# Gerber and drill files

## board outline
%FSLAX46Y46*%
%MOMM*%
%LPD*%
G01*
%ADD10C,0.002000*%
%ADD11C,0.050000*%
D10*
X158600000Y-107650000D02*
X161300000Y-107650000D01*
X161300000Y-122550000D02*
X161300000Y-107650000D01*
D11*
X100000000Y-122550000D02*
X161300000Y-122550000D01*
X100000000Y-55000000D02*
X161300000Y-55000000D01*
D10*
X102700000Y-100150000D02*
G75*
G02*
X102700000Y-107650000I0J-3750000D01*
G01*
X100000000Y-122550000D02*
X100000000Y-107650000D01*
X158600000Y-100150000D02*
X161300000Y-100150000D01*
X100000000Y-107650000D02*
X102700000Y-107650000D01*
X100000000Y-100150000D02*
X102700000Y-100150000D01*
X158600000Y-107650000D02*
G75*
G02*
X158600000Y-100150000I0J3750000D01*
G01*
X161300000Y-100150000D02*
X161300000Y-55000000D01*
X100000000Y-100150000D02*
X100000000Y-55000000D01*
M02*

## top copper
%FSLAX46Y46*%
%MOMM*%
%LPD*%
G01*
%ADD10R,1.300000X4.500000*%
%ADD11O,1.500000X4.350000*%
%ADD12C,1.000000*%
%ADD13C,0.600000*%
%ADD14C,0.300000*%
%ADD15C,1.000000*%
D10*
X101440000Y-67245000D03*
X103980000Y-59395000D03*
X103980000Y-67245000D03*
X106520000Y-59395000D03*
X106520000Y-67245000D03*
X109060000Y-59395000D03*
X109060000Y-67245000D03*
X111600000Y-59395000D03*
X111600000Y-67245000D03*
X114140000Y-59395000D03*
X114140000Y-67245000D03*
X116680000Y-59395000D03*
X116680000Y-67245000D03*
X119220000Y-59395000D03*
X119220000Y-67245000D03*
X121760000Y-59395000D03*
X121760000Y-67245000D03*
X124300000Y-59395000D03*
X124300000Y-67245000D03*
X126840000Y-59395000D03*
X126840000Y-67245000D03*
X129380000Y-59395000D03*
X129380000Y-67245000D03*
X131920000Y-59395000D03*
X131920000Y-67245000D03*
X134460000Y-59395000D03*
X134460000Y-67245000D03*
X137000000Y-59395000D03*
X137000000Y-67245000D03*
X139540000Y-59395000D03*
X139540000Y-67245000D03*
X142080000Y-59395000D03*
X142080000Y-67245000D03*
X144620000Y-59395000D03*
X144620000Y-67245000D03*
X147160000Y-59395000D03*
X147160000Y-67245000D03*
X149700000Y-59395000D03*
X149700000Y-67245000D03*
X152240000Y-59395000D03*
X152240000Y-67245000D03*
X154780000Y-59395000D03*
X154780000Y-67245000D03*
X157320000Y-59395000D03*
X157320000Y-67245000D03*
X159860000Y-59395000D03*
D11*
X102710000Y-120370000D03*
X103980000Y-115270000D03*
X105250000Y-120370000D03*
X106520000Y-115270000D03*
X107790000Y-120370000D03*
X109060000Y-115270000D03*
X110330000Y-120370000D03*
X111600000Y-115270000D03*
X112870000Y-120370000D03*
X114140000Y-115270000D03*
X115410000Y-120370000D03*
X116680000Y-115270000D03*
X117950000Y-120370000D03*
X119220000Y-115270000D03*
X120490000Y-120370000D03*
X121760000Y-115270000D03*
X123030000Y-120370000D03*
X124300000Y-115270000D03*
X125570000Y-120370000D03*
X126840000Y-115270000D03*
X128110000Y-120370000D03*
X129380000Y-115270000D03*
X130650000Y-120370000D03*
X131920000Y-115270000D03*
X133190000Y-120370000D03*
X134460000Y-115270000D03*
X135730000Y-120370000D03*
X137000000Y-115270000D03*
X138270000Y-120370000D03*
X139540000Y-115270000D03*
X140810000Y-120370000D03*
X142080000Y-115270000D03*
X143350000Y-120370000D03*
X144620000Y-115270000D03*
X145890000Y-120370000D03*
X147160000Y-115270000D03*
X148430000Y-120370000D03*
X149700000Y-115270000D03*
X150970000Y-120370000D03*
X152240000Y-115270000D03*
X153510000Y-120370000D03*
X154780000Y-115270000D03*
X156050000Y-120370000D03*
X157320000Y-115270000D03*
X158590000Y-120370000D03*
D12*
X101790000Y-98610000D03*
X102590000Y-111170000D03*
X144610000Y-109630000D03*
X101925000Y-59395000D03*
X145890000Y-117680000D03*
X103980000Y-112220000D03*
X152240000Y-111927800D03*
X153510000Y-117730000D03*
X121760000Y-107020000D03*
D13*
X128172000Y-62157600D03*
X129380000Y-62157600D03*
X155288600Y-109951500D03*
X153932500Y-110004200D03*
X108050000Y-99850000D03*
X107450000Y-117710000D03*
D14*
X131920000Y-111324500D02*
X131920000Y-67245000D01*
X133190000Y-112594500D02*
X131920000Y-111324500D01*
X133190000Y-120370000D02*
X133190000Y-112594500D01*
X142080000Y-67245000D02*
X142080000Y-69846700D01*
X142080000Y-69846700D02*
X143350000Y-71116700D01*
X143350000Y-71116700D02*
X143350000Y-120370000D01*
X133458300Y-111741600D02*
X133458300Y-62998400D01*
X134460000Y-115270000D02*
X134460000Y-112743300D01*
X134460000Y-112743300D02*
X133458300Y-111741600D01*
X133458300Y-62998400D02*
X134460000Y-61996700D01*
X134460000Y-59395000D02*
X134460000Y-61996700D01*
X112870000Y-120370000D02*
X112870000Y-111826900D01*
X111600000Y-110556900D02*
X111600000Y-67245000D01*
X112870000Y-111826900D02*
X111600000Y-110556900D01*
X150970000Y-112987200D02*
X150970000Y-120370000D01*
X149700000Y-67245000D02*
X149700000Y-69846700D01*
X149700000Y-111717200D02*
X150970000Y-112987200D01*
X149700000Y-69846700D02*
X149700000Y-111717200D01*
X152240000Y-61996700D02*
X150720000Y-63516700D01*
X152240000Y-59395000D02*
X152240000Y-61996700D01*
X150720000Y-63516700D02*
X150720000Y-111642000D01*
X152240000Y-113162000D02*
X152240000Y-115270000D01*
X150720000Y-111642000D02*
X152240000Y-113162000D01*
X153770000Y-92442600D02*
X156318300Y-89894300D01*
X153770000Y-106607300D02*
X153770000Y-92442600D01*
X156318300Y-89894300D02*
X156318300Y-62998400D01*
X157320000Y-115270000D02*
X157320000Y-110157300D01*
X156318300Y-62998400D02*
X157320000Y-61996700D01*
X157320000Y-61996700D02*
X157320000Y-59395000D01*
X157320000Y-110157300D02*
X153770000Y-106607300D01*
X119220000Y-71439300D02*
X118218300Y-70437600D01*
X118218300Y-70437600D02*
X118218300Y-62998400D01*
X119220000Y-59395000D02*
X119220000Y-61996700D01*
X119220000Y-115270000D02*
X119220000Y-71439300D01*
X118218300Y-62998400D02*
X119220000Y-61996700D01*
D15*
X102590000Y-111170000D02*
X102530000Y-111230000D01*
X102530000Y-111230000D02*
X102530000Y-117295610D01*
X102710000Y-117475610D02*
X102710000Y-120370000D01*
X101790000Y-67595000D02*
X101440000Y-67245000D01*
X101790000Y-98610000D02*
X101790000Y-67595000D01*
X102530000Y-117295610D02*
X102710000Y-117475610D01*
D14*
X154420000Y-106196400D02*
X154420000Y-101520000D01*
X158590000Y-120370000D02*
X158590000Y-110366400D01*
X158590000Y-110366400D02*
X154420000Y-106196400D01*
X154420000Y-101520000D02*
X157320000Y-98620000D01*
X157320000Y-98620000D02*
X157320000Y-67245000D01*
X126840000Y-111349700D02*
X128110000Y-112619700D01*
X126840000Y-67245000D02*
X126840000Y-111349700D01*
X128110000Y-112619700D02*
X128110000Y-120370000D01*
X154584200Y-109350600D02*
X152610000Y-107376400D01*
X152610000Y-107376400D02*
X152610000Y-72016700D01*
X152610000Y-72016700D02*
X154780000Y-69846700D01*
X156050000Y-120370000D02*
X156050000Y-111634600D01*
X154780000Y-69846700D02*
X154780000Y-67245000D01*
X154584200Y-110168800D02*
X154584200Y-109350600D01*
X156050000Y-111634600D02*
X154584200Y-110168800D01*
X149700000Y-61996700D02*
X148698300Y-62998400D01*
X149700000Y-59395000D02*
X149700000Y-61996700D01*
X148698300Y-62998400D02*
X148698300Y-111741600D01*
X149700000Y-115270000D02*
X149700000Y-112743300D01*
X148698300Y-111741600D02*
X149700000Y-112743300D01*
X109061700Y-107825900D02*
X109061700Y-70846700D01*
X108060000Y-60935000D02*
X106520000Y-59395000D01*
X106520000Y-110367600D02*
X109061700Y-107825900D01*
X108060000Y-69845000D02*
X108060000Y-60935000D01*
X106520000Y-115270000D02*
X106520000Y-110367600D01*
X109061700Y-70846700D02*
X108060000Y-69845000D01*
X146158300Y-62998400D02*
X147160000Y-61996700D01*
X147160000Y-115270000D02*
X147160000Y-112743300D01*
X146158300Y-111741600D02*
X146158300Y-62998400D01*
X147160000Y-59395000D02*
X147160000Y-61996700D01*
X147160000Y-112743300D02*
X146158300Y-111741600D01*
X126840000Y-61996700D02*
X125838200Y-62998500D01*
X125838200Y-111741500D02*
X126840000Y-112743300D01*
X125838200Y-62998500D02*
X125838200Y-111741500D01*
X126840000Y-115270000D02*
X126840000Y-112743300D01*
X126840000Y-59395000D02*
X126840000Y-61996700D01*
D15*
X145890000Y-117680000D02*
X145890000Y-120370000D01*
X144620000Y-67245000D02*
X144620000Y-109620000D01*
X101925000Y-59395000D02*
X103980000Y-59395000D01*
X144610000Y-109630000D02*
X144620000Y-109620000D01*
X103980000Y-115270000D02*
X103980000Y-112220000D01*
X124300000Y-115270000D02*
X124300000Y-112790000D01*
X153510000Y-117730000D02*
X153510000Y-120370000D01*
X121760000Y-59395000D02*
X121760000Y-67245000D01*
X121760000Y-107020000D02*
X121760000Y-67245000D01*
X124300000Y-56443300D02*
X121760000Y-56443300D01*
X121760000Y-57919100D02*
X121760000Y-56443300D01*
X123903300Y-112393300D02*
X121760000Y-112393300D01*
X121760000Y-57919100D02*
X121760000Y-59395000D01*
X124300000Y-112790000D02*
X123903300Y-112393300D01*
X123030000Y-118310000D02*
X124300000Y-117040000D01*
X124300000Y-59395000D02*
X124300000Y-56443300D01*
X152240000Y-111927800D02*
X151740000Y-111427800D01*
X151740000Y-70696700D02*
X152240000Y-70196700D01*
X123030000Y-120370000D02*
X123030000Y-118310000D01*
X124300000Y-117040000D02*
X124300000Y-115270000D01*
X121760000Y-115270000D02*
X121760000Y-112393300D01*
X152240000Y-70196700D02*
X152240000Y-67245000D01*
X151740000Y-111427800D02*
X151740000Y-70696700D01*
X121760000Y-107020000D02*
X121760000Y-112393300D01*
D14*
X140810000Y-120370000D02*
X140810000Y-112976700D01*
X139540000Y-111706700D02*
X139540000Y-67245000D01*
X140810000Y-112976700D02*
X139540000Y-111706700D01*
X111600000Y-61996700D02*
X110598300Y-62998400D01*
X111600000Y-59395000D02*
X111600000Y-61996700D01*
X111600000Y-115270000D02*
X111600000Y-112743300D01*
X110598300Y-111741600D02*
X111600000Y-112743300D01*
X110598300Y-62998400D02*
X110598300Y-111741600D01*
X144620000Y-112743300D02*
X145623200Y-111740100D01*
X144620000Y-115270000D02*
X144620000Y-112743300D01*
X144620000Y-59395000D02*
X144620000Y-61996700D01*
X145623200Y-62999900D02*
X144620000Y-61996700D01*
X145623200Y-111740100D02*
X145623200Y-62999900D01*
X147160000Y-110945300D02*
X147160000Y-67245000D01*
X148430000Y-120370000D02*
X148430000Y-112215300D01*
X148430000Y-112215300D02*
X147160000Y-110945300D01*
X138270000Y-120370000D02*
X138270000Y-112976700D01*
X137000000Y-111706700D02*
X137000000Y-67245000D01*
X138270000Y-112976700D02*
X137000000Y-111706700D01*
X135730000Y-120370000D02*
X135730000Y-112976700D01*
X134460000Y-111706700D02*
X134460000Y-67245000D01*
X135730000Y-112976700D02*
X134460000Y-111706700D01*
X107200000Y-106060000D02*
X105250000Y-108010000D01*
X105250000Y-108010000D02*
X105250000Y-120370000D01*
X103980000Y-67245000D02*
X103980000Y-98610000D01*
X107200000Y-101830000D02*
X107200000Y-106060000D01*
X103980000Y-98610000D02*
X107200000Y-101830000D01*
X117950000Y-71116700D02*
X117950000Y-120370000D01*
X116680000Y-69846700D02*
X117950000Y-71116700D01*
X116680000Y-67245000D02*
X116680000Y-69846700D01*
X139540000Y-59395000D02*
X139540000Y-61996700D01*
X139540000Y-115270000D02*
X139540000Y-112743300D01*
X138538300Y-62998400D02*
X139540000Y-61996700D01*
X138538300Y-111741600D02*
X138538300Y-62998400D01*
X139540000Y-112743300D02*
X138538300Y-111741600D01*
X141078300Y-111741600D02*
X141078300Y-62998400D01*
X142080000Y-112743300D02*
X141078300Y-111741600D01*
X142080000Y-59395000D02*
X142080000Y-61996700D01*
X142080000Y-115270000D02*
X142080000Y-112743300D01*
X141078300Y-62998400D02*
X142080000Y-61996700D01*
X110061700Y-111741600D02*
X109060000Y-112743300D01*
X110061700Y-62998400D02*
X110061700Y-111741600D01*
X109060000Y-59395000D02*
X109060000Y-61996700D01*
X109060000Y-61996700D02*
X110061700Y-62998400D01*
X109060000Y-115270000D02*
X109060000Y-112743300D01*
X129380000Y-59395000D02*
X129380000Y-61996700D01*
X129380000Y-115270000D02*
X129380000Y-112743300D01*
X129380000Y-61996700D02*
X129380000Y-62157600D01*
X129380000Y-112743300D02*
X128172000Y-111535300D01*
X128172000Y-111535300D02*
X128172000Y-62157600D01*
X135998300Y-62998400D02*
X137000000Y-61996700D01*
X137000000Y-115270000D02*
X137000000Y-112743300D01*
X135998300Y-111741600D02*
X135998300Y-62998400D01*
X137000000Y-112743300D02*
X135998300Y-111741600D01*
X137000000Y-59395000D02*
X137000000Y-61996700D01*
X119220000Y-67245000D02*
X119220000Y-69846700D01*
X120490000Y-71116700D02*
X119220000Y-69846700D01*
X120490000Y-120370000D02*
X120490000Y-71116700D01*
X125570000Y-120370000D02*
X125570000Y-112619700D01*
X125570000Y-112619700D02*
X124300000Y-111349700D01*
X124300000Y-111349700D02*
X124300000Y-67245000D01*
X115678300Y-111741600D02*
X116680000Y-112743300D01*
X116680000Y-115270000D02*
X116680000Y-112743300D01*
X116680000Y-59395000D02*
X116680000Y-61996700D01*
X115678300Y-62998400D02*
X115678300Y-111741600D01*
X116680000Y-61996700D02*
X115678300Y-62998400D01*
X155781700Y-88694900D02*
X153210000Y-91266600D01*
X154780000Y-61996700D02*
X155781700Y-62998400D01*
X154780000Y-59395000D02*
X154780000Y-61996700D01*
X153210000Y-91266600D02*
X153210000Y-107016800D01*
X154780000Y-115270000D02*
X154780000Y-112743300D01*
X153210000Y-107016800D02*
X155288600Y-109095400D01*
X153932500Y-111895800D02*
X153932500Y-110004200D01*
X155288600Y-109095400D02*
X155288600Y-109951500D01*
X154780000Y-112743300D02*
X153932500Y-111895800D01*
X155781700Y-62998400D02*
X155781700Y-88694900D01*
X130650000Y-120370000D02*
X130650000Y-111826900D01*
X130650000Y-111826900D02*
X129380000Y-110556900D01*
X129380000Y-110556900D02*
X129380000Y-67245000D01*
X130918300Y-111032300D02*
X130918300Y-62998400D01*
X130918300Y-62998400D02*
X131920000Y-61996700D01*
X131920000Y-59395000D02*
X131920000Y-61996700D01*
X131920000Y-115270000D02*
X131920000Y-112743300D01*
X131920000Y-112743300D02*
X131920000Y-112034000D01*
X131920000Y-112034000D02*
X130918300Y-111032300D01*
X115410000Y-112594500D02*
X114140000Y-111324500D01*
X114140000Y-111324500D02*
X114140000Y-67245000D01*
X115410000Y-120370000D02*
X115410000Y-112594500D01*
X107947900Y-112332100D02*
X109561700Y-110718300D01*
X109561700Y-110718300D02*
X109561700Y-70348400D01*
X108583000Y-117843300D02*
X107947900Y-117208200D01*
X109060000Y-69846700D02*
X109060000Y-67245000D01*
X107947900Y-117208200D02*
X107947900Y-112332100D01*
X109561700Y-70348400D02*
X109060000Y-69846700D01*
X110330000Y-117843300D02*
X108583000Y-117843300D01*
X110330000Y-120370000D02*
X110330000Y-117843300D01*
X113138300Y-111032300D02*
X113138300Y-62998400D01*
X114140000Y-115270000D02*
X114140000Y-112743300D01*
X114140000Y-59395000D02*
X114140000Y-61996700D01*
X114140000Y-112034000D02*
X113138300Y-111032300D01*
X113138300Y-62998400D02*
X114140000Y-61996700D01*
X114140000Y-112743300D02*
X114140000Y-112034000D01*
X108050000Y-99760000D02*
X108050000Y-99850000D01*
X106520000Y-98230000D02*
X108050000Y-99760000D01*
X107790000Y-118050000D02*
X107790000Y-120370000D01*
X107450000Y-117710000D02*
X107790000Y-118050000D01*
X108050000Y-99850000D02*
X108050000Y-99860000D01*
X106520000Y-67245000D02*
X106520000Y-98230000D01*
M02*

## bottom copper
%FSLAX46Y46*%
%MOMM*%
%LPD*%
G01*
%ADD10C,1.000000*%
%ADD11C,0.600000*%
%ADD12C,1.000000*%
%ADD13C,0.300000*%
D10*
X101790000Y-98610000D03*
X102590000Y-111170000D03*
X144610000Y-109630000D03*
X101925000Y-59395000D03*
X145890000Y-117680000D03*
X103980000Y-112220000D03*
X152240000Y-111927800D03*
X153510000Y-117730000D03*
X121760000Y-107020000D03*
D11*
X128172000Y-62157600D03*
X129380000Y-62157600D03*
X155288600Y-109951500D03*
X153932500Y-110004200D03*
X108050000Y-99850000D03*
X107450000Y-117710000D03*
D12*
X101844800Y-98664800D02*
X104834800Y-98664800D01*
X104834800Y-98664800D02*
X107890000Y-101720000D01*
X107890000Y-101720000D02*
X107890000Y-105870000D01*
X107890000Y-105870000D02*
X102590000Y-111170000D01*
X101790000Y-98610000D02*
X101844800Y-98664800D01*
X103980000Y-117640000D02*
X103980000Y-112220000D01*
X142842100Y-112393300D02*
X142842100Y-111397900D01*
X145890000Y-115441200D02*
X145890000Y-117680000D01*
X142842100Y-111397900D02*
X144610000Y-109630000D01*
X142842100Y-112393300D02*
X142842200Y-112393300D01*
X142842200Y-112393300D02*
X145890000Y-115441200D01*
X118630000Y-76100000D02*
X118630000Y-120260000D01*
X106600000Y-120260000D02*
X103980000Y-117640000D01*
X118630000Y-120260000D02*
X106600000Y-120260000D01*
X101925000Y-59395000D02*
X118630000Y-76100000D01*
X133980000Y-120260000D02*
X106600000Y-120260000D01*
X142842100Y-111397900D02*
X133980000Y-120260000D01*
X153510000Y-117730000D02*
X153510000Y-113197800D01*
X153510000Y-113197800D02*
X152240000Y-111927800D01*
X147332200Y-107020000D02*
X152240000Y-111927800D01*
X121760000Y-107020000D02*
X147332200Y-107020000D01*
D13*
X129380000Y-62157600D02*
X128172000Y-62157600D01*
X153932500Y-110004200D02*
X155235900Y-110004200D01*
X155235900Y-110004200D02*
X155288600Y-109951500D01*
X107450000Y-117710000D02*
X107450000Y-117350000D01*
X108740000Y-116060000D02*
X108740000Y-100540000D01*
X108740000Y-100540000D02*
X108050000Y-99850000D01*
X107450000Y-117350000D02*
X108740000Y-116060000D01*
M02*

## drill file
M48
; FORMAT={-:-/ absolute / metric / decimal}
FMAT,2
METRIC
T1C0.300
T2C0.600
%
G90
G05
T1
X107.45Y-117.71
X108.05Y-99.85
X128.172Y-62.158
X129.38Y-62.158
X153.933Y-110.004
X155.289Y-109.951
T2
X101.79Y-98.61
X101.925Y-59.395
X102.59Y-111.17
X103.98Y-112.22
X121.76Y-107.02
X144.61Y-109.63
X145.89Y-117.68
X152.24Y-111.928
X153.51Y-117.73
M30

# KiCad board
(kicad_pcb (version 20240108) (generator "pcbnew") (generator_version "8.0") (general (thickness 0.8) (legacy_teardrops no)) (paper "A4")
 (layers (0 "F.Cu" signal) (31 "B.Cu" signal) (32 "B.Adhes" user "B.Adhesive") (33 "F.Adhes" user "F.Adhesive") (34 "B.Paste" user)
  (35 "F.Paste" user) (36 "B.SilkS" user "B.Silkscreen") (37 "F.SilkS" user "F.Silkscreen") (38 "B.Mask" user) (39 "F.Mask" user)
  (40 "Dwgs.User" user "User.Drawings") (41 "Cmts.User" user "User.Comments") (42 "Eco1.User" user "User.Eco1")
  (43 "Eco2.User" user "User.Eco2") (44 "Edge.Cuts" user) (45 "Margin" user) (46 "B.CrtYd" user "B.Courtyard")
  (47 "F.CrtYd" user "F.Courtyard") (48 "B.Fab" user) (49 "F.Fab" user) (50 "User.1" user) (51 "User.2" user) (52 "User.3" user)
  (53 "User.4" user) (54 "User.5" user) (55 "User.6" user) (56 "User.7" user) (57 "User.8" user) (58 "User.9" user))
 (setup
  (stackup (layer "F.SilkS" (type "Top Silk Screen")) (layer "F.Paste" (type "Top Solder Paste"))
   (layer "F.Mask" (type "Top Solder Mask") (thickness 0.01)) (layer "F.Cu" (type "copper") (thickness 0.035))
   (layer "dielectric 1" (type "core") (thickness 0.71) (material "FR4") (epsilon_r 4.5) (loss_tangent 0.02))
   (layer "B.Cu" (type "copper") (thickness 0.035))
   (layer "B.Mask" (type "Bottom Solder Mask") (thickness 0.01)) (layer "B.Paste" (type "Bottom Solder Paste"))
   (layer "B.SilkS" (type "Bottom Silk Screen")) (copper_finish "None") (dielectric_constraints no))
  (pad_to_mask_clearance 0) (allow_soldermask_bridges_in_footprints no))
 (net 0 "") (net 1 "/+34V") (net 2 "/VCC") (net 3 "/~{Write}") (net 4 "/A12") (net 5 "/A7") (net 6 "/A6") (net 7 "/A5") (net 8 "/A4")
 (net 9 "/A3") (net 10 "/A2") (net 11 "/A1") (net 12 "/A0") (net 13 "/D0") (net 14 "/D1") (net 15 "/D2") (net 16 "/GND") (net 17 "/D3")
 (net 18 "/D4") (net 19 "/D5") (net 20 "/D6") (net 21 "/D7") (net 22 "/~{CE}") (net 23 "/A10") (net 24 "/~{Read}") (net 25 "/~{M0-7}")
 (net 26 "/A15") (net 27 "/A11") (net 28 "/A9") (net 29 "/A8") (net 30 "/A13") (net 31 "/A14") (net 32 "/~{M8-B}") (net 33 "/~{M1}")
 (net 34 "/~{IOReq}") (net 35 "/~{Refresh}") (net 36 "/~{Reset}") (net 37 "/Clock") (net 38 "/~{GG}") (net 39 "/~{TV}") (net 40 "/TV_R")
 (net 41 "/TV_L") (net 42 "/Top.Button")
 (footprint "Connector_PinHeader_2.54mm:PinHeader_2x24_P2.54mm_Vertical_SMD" (layer "F.Cu") (at 130.65 63.32 90)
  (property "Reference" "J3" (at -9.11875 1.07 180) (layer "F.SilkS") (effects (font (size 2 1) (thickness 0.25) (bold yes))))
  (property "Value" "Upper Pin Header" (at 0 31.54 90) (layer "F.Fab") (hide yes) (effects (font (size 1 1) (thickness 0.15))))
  (pad "1" smd rect (at -3.925 -29.21 90) (size 4.5 1.3) (layers "F.Cu" "F.Paste" "F.Mask") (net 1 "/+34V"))
  (pad "2" smd rect (at 3.925 -26.67 90) (size 4.5 1.3) (layers "F.Cu" "F.Paste" "F.Mask") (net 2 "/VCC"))
  (pad "3" smd rect (at -3.925 -26.67 90) (size 4.5 1.3) (layers "F.Cu" "F.Paste" "F.Mask") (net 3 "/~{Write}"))
  (pad "4" smd rect (at 3.925 -24.13 90) (size 4.5 1.3) (layers "F.Cu" "F.Paste" "F.Mask") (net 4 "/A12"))
  (pad "5" smd rect (at -3.925 -24.13 90) (size 4.5 1.3) (layers "F.Cu" "F.Paste" "F.Mask") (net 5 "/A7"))
  (pad "6" smd rect (at 3.925 -21.59 90) (size 4.5 1.3) (layers "F.Cu" "F.Paste" "F.Mask") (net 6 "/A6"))
  (pad "7" smd rect (at -3.925 -21.59 90) (size 4.5 1.3) (layers "F.Cu" "F.Paste" "F.Mask") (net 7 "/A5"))
  (pad "8" smd rect (at 3.925 -19.05 90) (size 4.5 1.3) (layers "F.Cu" "F.Paste" "F.Mask") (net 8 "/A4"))
  (pad "9" smd rect (at -3.925 -19.05 90) (size 4.5 1.3) (layers "F.Cu" "F.Paste" "F.Mask") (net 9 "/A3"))
  (pad "10" smd rect (at 3.925 -16.51 90) (size 4.5 1.3) (layers "F.Cu" "F.Paste" "F.Mask") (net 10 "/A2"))
  (pad "11" smd rect (at -3.925 -16.51 90) (size 4.5 1.3) (layers "F.Cu" "F.Paste" "F.Mask") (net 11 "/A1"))
  (pad "12" smd rect (at 3.925 -13.97 90) (size 4.5 1.3) (layers "F.Cu" "F.Paste" "F.Mask") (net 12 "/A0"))
  (pad "13" smd rect (at -3.925 -13.97 90) (size 4.5 1.3) (layers "F.Cu" "F.Paste" "F.Mask") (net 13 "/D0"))
  (pad "14" smd rect (at 3.925 -11.43 90) (size 4.5 1.3) (layers "F.Cu" "F.Paste" "F.Mask") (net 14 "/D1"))
  (pad "15" smd rect (at -3.925 -11.43 90) (size 4.5 1.3) (layers "F.Cu" "F.Paste" "F.Mask") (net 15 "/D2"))
  (pad "16" smd rect (at 3.925 -8.89 90) (size 4.5 1.3) (layers "F.Cu" "F.Paste" "F.Mask") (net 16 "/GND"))
  (pad "17" smd rect (at -3.925 -8.89 90) (size 4.5 1.3) (layers "F.Cu" "F.Paste" "F.Mask") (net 16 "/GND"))
  (pad "18" smd rect (at 3.925 -6.35 90) (size 4.5 1.3) (layers "F.Cu" "F.Paste" "F.Mask") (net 16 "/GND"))
  (pad "19" smd rect (at -3.925 -6.35 90) (size 4.5 1.3) (layers "F.Cu" "F.Paste" "F.Mask") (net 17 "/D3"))
  (pad "20" smd rect (at 3.925 -3.81 90) (size 4.5 1.3) (layers "F.Cu" "F.Paste" "F.Mask") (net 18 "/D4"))
  (pad "21" smd rect (at -3.925 -3.81 90) (size 4.5 1.3) (layers "F.Cu" "F.Paste" "F.Mask") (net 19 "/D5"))
  (pad "22" smd rect (at 3.925 -1.27 90) (size 4.5 1.3) (layers "F.Cu" "F.Paste" "F.Mask") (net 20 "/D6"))
  (pad "23" smd rect (at -3.925 -1.27 90) (size 4.5 1.3) (layers "F.Cu" "F.Paste" "F.Mask") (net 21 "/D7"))
  (pad "24" smd rect (at 3.925 1.27 90) (size 4.5 1.3) (layers "F.Cu" "F.Paste" "F.Mask") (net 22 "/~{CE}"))
  (pad "25" smd rect (at -3.925 1.27 90) (size 4.5 1.3) (layers "F.Cu" "F.Paste" "F.Mask") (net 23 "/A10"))
  (pad "26" smd rect (at 3.925 3.81 90) (size 4.5 1.3) (layers "F.Cu" "F.Paste" "F.Mask") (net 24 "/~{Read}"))
  (pad "27" smd rect (at -3.925 3.81 90) (size 4.5 1.3) (layers "F.Cu" "F.Paste" "F.Mask") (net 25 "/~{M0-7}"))
  (pad "28" smd rect (at 3.925 6.35 90) (size 4.5 1.3) (layers "F.Cu" "F.Paste" "F.Mask") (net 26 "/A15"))
  (pad "29" smd rect (at -3.925 6.35 90) (size 4.5 1.3) (layers "F.Cu" "F.Paste" "F.Mask") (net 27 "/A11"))
  (pad "30" smd rect (at 3.925 8.89 90) (size 4.5 1.3) (layers "F.Cu" "F.Paste" "F.Mask") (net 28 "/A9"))
  (pad "31" smd rect (at -3.925 8.89 90) (size 4.5 1.3) (layers "F.Cu" "F.Paste" "F.Mask") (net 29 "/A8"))
  (pad "32" smd rect (at 3.925 11.43 90) (size 4.5 1.3) (layers "F.Cu" "F.Paste" "F.Mask") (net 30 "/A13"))
  (pad "33" smd rect (at -3.925 11.43 90) (size 4.5 1.3) (layers "F.Cu" "F.Paste" "F.Mask") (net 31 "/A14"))
  (pad "34" smd rect (at 3.925 13.97 90) (size 4.5 1.3) (layers "F.Cu" "F.Paste" "F.Mask") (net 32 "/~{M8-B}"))
  (pad "35" smd rect (at -3.925 13.97 90) (size 4.5 1.3) (layers "F.Cu" "F.Paste" "F.Mask") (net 2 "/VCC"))
  (pad "36" smd rect (at 3.925 16.51 90) (size 4.5 1.3) (layers "F.Cu" "F.Paste" "F.Mask") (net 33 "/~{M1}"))
  (pad "37" smd rect (at -3.925 16.51 90) (size 4.5 1.3) (layers "F.Cu" "F.Paste" "F.Mask") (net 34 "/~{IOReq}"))
  (pad "38" smd rect (at 3.925 19.05 90) (size 4.5 1.3) (layers "F.Cu" "F.Paste" "F.Mask") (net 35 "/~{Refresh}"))
  (pad "39" smd rect (at -3.925 19.05 90) (size 4.5 1.3) (layers "F.Cu" "F.Paste" "F.Mask") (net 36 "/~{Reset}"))
  (pad "40" smd rect (at 3.925 21.59 90) (size 4.5 1.3) (layers "F.Cu" "F.Paste" "F.Mask") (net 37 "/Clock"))
  (pad "41" smd rect (at -3.925 21.59 90) (size 4.5 1.3) (layers "F.Cu" "F.Paste" "F.Mask") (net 16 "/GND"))
  (pad "42" smd rect (at 3.925 24.13 90) (size 4.5 1.3) (layers "F.Cu" "F.Paste" "F.Mask") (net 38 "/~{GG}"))
  (pad "43" smd rect (at -3.925 24.13 90) (size 4.5 1.3) (layers "F.Cu" "F.Paste" "F.Mask") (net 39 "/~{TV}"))
  (pad "44" smd rect (at 3.925 26.67 90) (size 4.5 1.3) (layers "F.Cu" "F.Paste" "F.Mask") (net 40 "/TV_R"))
  (pad "45" smd rect (at -3.925 26.67 90) (size 4.5 1.3) (layers "F.Cu" "F.Paste" "F.Mask") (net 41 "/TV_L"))
  (pad "46" smd rect (at 3.925 29.21 90) (size 4.5 1.3) (layers "F.Cu" "F.Paste" "F.Mask") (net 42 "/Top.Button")))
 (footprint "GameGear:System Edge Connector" (layer "F.Cu") (at 130.65 117.82)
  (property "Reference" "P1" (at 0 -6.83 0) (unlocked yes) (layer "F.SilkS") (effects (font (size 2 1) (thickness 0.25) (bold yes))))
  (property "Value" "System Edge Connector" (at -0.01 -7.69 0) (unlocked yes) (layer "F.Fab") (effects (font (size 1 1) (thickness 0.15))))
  (pad "1" smd oval (at -27.94 2.55) (size 1.5 4.35) (layers "F.Cu" "F.Mask") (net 1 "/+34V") (thermal_bridge_angle 45))
  (pad "2" smd oval (at -26.67 -2.55) (size 1.5 4.35) (layers "F.Cu" "F.Mask") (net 2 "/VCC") (thermal_bridge_angle 45))
  (pad "3" smd oval (at -25.4 2.55) (size 1.5 4.35) (layers "F.Cu" "F.Mask") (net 3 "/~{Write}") (thermal_bridge_angle 45))
  (pad "4" smd oval (at -24.13 -2.55) (size 1.5 4.35) (layers "F.Cu" "F.Mask") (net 4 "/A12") (thermal_bridge_angle 45))
  (pad "5" smd oval (at -22.86 2.55) (size 1.5 4.35) (layers "F.Cu" "F.Mask") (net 5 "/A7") (thermal_bridge_angle 45))
  (pad "6" smd oval (at -21.59 -2.55) (size 1.5 4.35) (layers "F.Cu" "F.Mask") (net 6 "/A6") (thermal_bridge_angle 45))
  (pad "7" smd oval (at -20.32 2.55) (size 1.5 4.35) (layers "F.Cu" "F.Mask") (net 7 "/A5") (thermal_bridge_angle 45))
  (pad "8" smd oval (at -19.05 -2.55) (size 1.5 4.35) (layers "F.Cu" "F.Mask") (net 8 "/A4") (thermal_bridge_angle 45))
  (pad "9" smd oval (at -17.78 2.55) (size 1.5 4.35) (layers "F.Cu" "F.Mask") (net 9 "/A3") (thermal_bridge_angle 45))
  (pad "10" smd oval (at -16.51 -2.55) (size 1.5 4.35) (layers "F.Cu" "F.Mask") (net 10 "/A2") (thermal_bridge_angle 45))
  (pad "11" smd oval (at -15.24 2.55) (size 1.5 4.35) (layers "F.Cu" "F.Mask") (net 11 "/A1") (thermal_bridge_angle 45))
  (pad "12" smd oval (at -13.97 -2.55) (size 1.5 4.35) (layers "F.Cu" "F.Mask") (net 12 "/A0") (thermal_bridge_angle 45))
  (pad "13" smd oval (at -12.7 2.55) (size 1.5 4.35) (layers "F.Cu" "F.Mask") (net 13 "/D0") (thermal_bridge_angle 45))
  (pad "14" smd oval (at -11.43 -2.55) (size 1.5 4.35) (layers "F.Cu" "F.Mask") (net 14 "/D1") (thermal_bridge_angle 45))
  (pad "15" smd oval (at -10.16 2.55) (size 1.5 4.35) (layers "F.Cu" "F.Mask") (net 15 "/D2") (thermal_bridge_angle 45))
  (pad "16" smd oval (at -8.89 -2.55) (size 1.5 4.35) (layers "F.Cu" "F.Mask") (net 16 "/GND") (thermal_bridge_angle 45))
  (pad "17" smd oval (at -7.62 2.55) (size 1.5 4.35) (layers "F.Cu" "F.Mask") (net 16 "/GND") (thermal_bridge_angle 45))
  (pad "18" smd oval (at -6.35 -2.55) (size 1.5 4.35) (layers "F.Cu" "F.Mask") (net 16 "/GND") (thermal_bridge_angle 45))
  (pad "19" smd oval (at -5.08 2.55) (size 1.5 4.35) (layers "F.Cu" "F.Mask") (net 17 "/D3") (thermal_bridge_angle 45))
  (pad "20" smd oval (at -3.81 -2.55) (size 1.5 4.35) (layers "F.Cu" "F.Mask") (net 18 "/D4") (thermal_bridge_angle 45))
  (pad "21" smd oval (at -2.54 2.55) (size 1.5 4.35) (layers "F.Cu" "F.Mask") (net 19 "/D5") (thermal_bridge_angle 45))
  (pad "22" smd oval (at -1.27 -2.55) (size 1.5 4.35) (layers "F.Cu" "F.Mask") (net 20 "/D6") (thermal_bridge_angle 45))
  (pad "23" smd oval (at 0 2.55) (size 1.5 4.35) (layers "F.Cu" "F.Mask") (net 21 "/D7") (thermal_bridge_angle 45))
  (pad "24" smd oval (at 1.27 -2.55) (size 1.5 4.35) (layers "F.Cu" "F.Mask") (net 22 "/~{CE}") (thermal_bridge_angle 45))
  (pad "25" smd oval (at 2.54 2.55) (size 1.5 4.35) (layers "F.Cu" "F.Mask") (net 23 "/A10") (thermal_bridge_angle 45))
  (pad "26" smd oval (at 3.81 -2.55) (size 1.5 4.35) (layers "F.Cu" "F.Mask") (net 24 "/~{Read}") (thermal_bridge_angle 45))
  (pad "27" smd oval (at 5.08 2.55) (size 1.5 4.35) (layers "F.Cu" "F.Mask") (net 25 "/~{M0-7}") (thermal_bridge_angle 45))
  (pad "28" smd oval (at 6.35 -2.55) (size 1.5 4.35) (layers "F.Cu" "F.Mask") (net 26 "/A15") (thermal_bridge_angle 45))
  (pad "29" smd oval (at 7.62 2.55) (size 1.5 4.35) (layers "F.Cu" "F.Mask") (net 27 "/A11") (thermal_bridge_angle 45))
  (pad "30" smd oval (at 8.89 -2.55) (size 1.5 4.35) (layers "F.Cu" "F.Mask") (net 28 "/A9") (thermal_bridge_angle 45))
  (pad "31" smd oval (at 10.16 2.55) (size 1.5 4.35) (layers "F.Cu" "F.Mask") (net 29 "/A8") (thermal_bridge_angle 45))
  (pad "32" smd oval (at 11.43 -2.55) (size 1.5 4.35) (layers "F.Cu" "F.Mask") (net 30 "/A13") (thermal_bridge_angle 45))
  (pad "33" smd oval (at 12.7 2.55) (size 1.5 4.35) (layers "F.Cu" "F.Mask") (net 31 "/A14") (thermal_bridge_angle 45))
  (pad "34" smd oval (at 13.97 -2.55) (size 1.5 4.35) (layers "F.Cu" "F.Mask") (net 32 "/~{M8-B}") (thermal_bridge_angle 45))
  (pad "35" smd oval (at 15.24 2.55) (size 1.5 4.35) (layers "F.Cu" "F.Mask") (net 2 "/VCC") (thermal_bridge_angle 45))
  (pad "36" smd oval (at 16.51 -2.55) (size 1.5 4.35) (layers "F.Cu" "F.Mask") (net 33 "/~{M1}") (thermal_bridge_angle 45))
  (pad "37" smd oval (at 17.78 2.55) (size 1.5 4.35) (layers "F.Cu" "F.Mask") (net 34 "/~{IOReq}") (thermal_bridge_angle 45))
  (pad "38" smd oval (at 19.05 -2.55) (size 1.5 4.35) (layers "F.Cu" "F.Mask") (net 35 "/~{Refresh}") (thermal_bridge_angle 45))
  (pad "39" smd oval (at 20.32 2.55) (size 1.5 4.35) (layers "F.Cu" "F.Mask") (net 36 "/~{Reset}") (thermal_bridge_angle 45))
  (pad "40" smd oval (at 21.59 -2.55) (size 1.5 4.35) (layers "F.Cu" "F.Mask") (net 37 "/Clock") (thermal_bridge_angle 45))
  (pad "41" smd oval (at 22.86 2.55) (size 1.5 4.35) (layers "F.Cu" "F.Mask") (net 16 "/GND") (thermal_bridge_angle 45))
  (pad "42" smd oval (at 24.13 -2.55) (size 1.5 4.35) (layers "F.Cu" "F.Mask") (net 38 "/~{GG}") (thermal_bridge_angle 45))
  (pad "43" smd oval (at 25.4 2.55) (size 1.5 4.35) (layers "F.Cu" "F.Mask") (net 39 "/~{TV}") (thermal_bridge_angle 45))
  (pad "44" smd oval (at 26.67 -2.55) (size 1.5 4.35) (layers "F.Cu" "F.Mask") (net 40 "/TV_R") (thermal_bridge_angle 45))
  (pad "45" smd oval (at 27.94 2.55) (size 1.5 4.35) (layers "F.Cu" "F.Mask") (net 41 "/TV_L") (thermal_bridge_angle 45)))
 (gr_line (start 158.6 107.65) (end 161.3 107.65) (stroke (width 0.002) (type default)) (layer "Edge.Cuts"))
 (gr_line (start 161.3 122.55) (end 161.3 107.65) (stroke (width 0.002) (type default)) (layer "Edge.Cuts"))
 (gr_line (start 100 122.55) (end 161.3 122.55) (stroke (width 0.05) (type default)) (layer "Edge.Cuts"))
 (gr_line (start 100 55) (end 161.3 55) (stroke (width 0.05) (type default)) (layer "Edge.Cuts"))
 (gr_arc (start 102.7 100.15) (mid 106.45 103.9) (end 102.7 107.65) (stroke (width 0.002) (type default)) (layer "Edge.Cuts"))
 (gr_line (start 100 122.55) (end 100 107.65) (stroke (width 0.002) (type default)) (layer "Edge.Cuts"))
 (gr_line (start 158.6 100.15) (end 161.3 100.15) (stroke (width 0.002) (type default)) (layer "Edge.Cuts"))
 (gr_line (start 100 107.65) (end 102.7 107.65) (stroke (width 0.002) (type default)) (layer "Edge.Cuts"))
 (gr_line (start 100 100.15) (end 102.7 100.15) (stroke (width 0.002) (type default)) (layer "Edge.Cuts"))
 (gr_arc (start 158.6 107.65) (mid 154.85 103.9) (end 158.6 100.15) (stroke (width 0.002) (type default)) (layer "Edge.Cuts"))
 (gr_line (start 161.3 100.15) (end 161.3 55) (stroke (width 0.002) (type default)) (layer "Edge.Cuts"))
 (gr_line (start 100 100.15) (end 100 55) (stroke (width 0.002) (type default)) (layer "Edge.Cuts"))
 (segment (start 131.92 111.3245) (end 131.92 67.245) (width 0.3) (layer "F.Cu") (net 23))
 (segment (start 133.19 112.5945) (end 131.92 111.3245) (width 0.3) (layer "F.Cu") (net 23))
 (segment (start 133.19 120.37) (end 133.19 112.5945) (width 0.3) (layer "F.Cu") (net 23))
 (segment (start 142.08 67.245) (end 142.08 69.8467) (width 0.3) (layer "F.Cu") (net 31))
 (segment (start 142.08 69.8467) (end 143.35 71.1167) (width 0.3) (layer "F.Cu") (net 31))
 (segment (start 143.35 71.1167) (end 143.35 120.37) (width 0.3) (layer "F.Cu") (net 31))
 (segment (start 133.4583 111.7416) (end 133.4583 62.9984) (width 0.3) (layer "F.Cu") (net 24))
 (segment (start 134.46 115.27) (end 134.46 112.7433) (width 0.3) (layer "F.Cu") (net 24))
 (segment (start 134.46 112.7433) (end 133.4583 111.7416) (width 0.3) (layer "F.Cu") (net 24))
 (segment (start 133.4583 62.9984) (end 134.46 61.9967) (width 0.3) (layer "F.Cu") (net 24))
 (segment (start 134.46 59.395) (end 134.46 61.9967) (width 0.3) (layer "F.Cu") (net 24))
 (segment (start 112.87 120.37) (end 112.87 111.8269) (width 0.3) (layer "F.Cu") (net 9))
 (segment (start 111.6 110.5569) (end 111.6 67.245) (width 0.3) (layer "F.Cu") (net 9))
 (segment (start 112.87 111.8269) (end 111.6 110.5569) (width 0.3) (layer "F.Cu") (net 9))
 (segment (start 150.97 112.9872) (end 150.97 120.37) (width 0.3) (layer "F.Cu") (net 36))
 (segment (start 149.7 67.245) (end 149.7 69.8467) (width 0.3) (layer "F.Cu") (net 36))
 (segment (start 149.7 111.7172) (end 150.97 112.9872) (width 0.3) (layer "F.Cu") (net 36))
 (segment (start 149.7 69.8467) (end 149.7 111.7172) (width 0.3) (layer "F.Cu") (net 36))
 (segment (start 152.24 61.9967) (end 150.72 63.5167) (width 0.3) (layer "F.Cu") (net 37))
 (segment (start 152.24 59.395) (end 152.24 61.9967) (width 0.3) (layer "F.Cu") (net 37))
 (segment (start 150.72 63.5167) (end 150.72 111.642) (width 0.3) (layer "F.Cu") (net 37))
 (segment (start 152.24 113.162) (end 152.24 115.27) (width 0.3) (layer "F.Cu") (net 37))
 (segment (start 150.72 111.642) (end 152.24 113.162) (width 0.3) (layer "F.Cu") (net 37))
 (segment (start 153.77 92.4426) (end 156.3183 89.8943) (width 0.3) (layer "F.Cu") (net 40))
 (segment (start 153.77 106.6073) (end 153.77 92.4426) (width 0.3) (layer "F.Cu") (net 40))
 (segment (start 156.3183 89.8943) (end 156.3183 62.9984) (width 0.3) (layer "F.Cu") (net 40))
 (segment (start 157.32 115.27) (end 157.32 110.1573) (width 0.3) (layer "F.Cu") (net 40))
 (segment (start 156.3183 62.9984) (end 157.32 61.9967) (width 0.3) (layer "F.Cu") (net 40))
 (segment (start 157.32 61.9967) (end 157.32 59.395) (width 0.3) (layer "F.Cu") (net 40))
 (segment (start 157.32 110.1573) (end 153.77 106.6073) (width 0.3) (layer "F.Cu") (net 40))
 (segment (start 119.22 71.4393) (end 118.2183 70.4376) (width 0.3) (layer "F.Cu") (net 14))
 (segment (start 118.2183 70.4376) (end 118.2183 62.9984) (width 0.3) (layer "F.Cu") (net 14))
 (segment (start 119.22 59.395) (end 119.22 61.9967) (width 0.3) (layer "F.Cu") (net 14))
 (segment (start 119.22 115.27) (end 119.22 71.4393) (width 0.3) (layer "F.Cu") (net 14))
 (segment (start 118.2183 62.9984) (end 119.22 61.9967) (width 0.3) (layer "F.Cu") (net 14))
 (segment (start 102.59 111.17) (end 102.53 111.23) (width 1) (layer "F.Cu") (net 1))
 (segment (start 102.53 111.23) (end 102.53 117.29561) (width 1) (layer "F.Cu") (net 1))
 (segment (start 102.71 117.47561) (end 102.71 120.37) (width 1) (layer "F.Cu") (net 1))
 (segment (start 101.79 67.595) (end 101.44 67.245) (width 1) (layer "F.Cu") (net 1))
 (segment (start 101.79 98.61) (end 101.79 67.595) (width 1) (layer "F.Cu") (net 1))
 (segment (start 102.53 117.29561) (end 102.71 117.47561) (width 1) (layer "F.Cu") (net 1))
 (via (at 101.79 98.61) (size 1) (drill 0.6) (layers "F.Cu" "B.Cu") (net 1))
 (via (at 102.59 111.17) (size 1) (drill 0.6) (layers "F.Cu" "B.Cu") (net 1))
 (segment (start 101.8448 98.6648) (end 104.8348 98.6648) (width 1) (layer "B.Cu") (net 1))
 (segment (start 104.8348 98.6648) (end 107.89 101.72) (width 1) (layer "B.Cu") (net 1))
 (segment (start 107.89 101.72) (end 107.89 105.87) (width 1) (layer "B.Cu") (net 1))
 (segment (start 107.89 105.87) (end 102.59 111.17) (width 1) (layer "B.Cu") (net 1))
 (segment (start 101.79 98.61) (end 101.8448 98.6648) (width 1) (layer "B.Cu") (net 1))
 (segment (start 154.42 106.1964) (end 154.42 101.52) (width 0.3) (layer "F.Cu") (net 41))
 (segment (start 158.59 120.37) (end 158.59 110.3664) (width 0.3) (layer "F.Cu") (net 41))
 (segment (start 158.59 110.3664) (end 154.42 106.1964) (width 0.3) (layer "F.Cu") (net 41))
 (segment (start 154.42 101.52) (end 157.32 98.62) (width 0.3) (layer "F.Cu") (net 41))
 (segment (start 157.32 98.62) (end 157.32 67.245) (width 0.3) (layer "F.Cu") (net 41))
 (segment (start 126.84 111.3497) (end 128.11 112.6197) (width 0.3) (layer "F.Cu") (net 19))
 (segment (start 126.84 67.245) (end 126.84 111.3497) (width 0.3) (layer "F.Cu") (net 19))
 (segment (start 128.11 112.6197) (end 128.11 120.37) (width 0.3) (layer "F.Cu") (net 19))
 (segment (start 154.5842 109.3506) (end 152.61 107.3764) (width 0.3) (layer "F.Cu") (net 39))
 (segment (start 152.61 107.3764) (end 152.61 72.0167) (width 0.3) (layer "F.Cu") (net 39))
 (segment (start 152.61 72.0167) (end 154.78 69.8467) (width 0.3) (layer "F.Cu") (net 39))
 (segment (start 156.05 120.37) (end 156.05 111.6346) (width 0.3) (layer "F.Cu") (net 39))
 (segment (start 154.78 69.8467) (end 154.78 67.245) (width 0.3) (layer "F.Cu") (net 39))
 (segment (start 154.5842 110.1688) (end 154.5842 109.3506) (width 0.3) (layer "F.Cu") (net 39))
 (segment (start 156.05 111.6346) (end 154.5842 110.1688) (width 0.3) (layer "F.Cu") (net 39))
 (segment (start 149.7 61.9967) (end 148.6983 62.9984) (width 0.3) (layer "F.Cu") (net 35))
 (segment (start 149.7 59.395) (end 149.7 61.9967) (width 0.3) (layer "F.Cu") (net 35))
 (segment (start 148.6983 62.9984) (end 148.6983 111.7416) (width 0.3) (layer "F.Cu") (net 35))
 (segment (start 149.7 115.27) (end 149.7 112.7433) (width 0.3) (layer "F.Cu") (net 35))
 (segment (start 148.6983 111.7416) (end 149.7 112.7433) (width 0.3) (layer "F.Cu") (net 35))
 (segment (start 109.0617 107.8259) (end 109.0617 70.8467) (width 0.3) (layer "F.Cu") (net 4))
 (segment (start 108.06 60.935) (end 106.52 59.395) (width 0.3) (layer "F.Cu") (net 4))
 (segment (start 106.52 110.3676) (end 109.0617 107.8259) (width 0.3) (layer "F.Cu") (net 4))
 (segment (start 108.06 69.845) (end 108.06 60.935) (width 0.3) (layer "F.Cu") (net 4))
 (segment (start 106.52 115.27) (end 106.52 110.3676) (width 0.3) (layer "F.Cu") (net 4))
 (segment (start 109.0617 70.8467) (end 108.06 69.845) (width 0.3) (layer "F.Cu") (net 4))
 (segment (start 146.1583 62.9984) (end 147.16 61.9967) (width 0.3) (layer "F.Cu") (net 33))
 (segment (start 147.16 115.27) (end 147.16 112.7433) (width 0.3) (layer "F.Cu") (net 33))
 (segment (start 146.1583 111.7416) (end 146.1583 62.9984) (width 0.3) (layer "F.Cu") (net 33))
 (segment (start 147.16 59.395) (end 147.16 61.9967) (width 0.3) (layer "F.Cu") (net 33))
 (segment (start 147.16 112.7433) (end 146.1583 111.7416) (width 0.3) (layer "F.Cu") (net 33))
 (segment (start 126.84 61.9967) (end 125.8382 62.9985) (width 0.3) (layer "F.Cu") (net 18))
 (segment (start 125.8382 111.7415) (end 126.84 112.7433) (width 0.3) (layer "F.Cu") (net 18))
 (segment (start 125.8382 62.9985) (end 125.8382 111.7415) (width 0.3) (layer "F.Cu") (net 18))
 (segment (start 126.84 115.27) (end 126.84 112.7433) (width 0.3) (layer "F.Cu") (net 18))
 (segment (start 126.84 59.395) (end 126.84 61.9967) (width 0.3) (layer "F.Cu") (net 18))
 (segment (start 145.89 117.68) (end 145.89 120.37) (width 1) (layer "F.Cu") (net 2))
 (segment (start 144.62 67.245) (end 144.62 109.62) (width 1) (layer "F.Cu") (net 2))
 (segment (start 101.925 59.395) (end 103.98 59.395) (width 1) (layer "F.Cu") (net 2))
 (segment (start 144.61 109.63) (end 144.62 109.62) (width 1) (layer "F.Cu") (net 2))
 (segment (start 103.98 115.27) (end 103.98 112.22) (width 1) (layer "F.Cu") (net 2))
 (via (at 144.61 109.63) (size 1) (drill 0.6) (layers "F.Cu" "B.Cu") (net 2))
 (via (at 101.925 59.395) (size 1) (drill 0.6) (layers "F.Cu" "B.Cu") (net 2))
 (via (at 145.89 117.68) (size 1) (drill 0.6) (layers "F.Cu" "B.Cu") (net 2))
 (via (at 103.98 112.22) (size 1) (drill 0.6) (layers "F.Cu" "B.Cu") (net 2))
 (segment (start 103.98 117.64) (end 103.98 112.22) (width 1) (layer "B.Cu") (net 2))
 (segment (start 142.8421 112.3933) (end 142.8421 111.3979) (width 1) (layer "B.Cu") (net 2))
 (segment (start 145.89 115.4412) (end 145.89 117.68) (width 1) (layer "B.Cu") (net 2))
 (segment (start 142.8421 111.3979) (end 144.61 109.63) (width 1) (layer "B.Cu") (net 2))
 (segment (start 142.8421 112.3933) (end 142.8422 112.3933) (width 1) (layer "B.Cu") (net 2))
 (segment (start 142.8422 112.3933) (end 145.89 115.4412) (width 1) (layer "B.Cu") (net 2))
 (segment (start 118.63 76.1) (end 118.63 120.26) (width 1) (layer "B.Cu") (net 2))
 (segment (start 106.6 120.26) (end 103.98 117.64) (width 1) (layer "B.Cu") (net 2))
 (segment (start 118.63 120.26) (end 106.6 120.26) (width 1) (layer "B.Cu") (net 2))
 (segment (start 101.925 59.395) (end 118.63 76.1) (width 1) (layer "B.Cu") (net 2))
 (segment (start 133.98 120.26) (end 106.6 120.26) (width 1) (layer "B.Cu") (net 2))
 (segment (start 142.8421 111.3979) (end 133.98 120.26) (width 1) (layer "B.Cu") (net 2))
 (segment (start 124.3 115.27) (end 124.3 112.79) (width 1) (layer "F.Cu") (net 16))
 (segment (start 153.51 117.73) (end 153.51 120.37) (width 1) (layer "F.Cu") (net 16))
 (segment (start 121.76 59.395) (end 121.76 67.245) (width 1) (layer "F.Cu") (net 16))
 (segment (start 121.76 107.02) (end 121.76 67.245) (width 1) (layer "F.Cu") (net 16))
 (segment (start 124.3 56.4433) (end 121.76 56.4433) (width 1) (layer "F.Cu") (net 16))
 (segment (start 121.76 57.9191) (end 121.76 56.4433) (width 1) (layer "F.Cu") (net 16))
 (segment (start 123.9033 112.3933) (end 121.76 112.3933) (width 1) (layer "F.Cu") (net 16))
 (segment (start 121.76 57.9191) (end 121.76 59.395) (width 1) (layer "F.Cu") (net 16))
 (segment (start 124.3 112.79) (end 123.9033 112.3933) (width 1) (layer "F.Cu") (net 16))
 (segment (start 123.03 118.31) (end 124.3 117.04) (width 1) (layer "F.Cu") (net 16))
 (segment (start 124.3 59.395) (end 124.3 56.4433) (width 1) (layer "F.Cu") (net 16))
 (segment (start 152.24 111.9278) (end 151.74 111.4278) (width 1) (layer "F.Cu") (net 16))
 (segment (start 151.74 70.6967) (end 152.24 70.1967) (width 1) (layer "F.Cu") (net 16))
 (segment (start 123.03 120.37) (end 123.03 118.31) (width 1) (layer "F.Cu") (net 16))
 (segment (start 124.3 117.04) (end 124.3 115.27) (width 1) (layer "F.Cu") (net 16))
 (segment (start 121.76 115.27) (end 121.76 112.3933) (width 1) (layer "F.Cu") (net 16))
 (segment (start 152.24 70.1967) (end 152.24 67.245) (width 1) (layer "F.Cu") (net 16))
 (segment (start 151.74 111.4278) (end 151.74 70.6967) (width 1) (layer "F.Cu") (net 16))
 (segment (start 121.76 107.02) (end 121.76 112.3933) (width 1) (layer "F.Cu") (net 16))
 (via (at 152.24 111.9278) (size 1) (drill 0.6) (layers "F.Cu" "B.Cu") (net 16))
 (via (at 153.51 117.73) (size 1) (drill 0.6) (layers "F.Cu" "B.Cu") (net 16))
 (via (at 121.76 107.02) (size 1) (drill 0.6) (layers "F.Cu" "B.Cu") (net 16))
 (segment (start 153.51 117.73) (end 153.51 113.1978) (width 1) (layer "B.Cu") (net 16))
 (segment (start 153.51 113.1978) (end 152.24 111.9278) (width 1) (layer "B.Cu") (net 16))
 (segment (start 147.3322 107.02) (end 152.24 111.9278) (width 1) (layer "B.Cu") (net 16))
 (segment (start 121.76 107.02) (end 147.3322 107.02) (width 1) (layer "B.Cu") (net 16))
 (segment (start 140.81 120.37) (end 140.81 112.9767) (width 0.3) (layer "F.Cu") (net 29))
 (segment (start 139.54 111.7067) (end 139.54 67.245) (width 0.3) (layer "F.Cu") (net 29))
 (segment (start 140.81 112.9767) (end 139.54 111.7067) (width 0.3) (layer "F.Cu") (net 29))
 (segment (start 111.6 61.9967) (end 110.5983 62.9984) (width 0.3) (layer "F.Cu") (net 8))
 (segment (start 111.6 59.395) (end 111.6 61.9967) (width 0.3) (layer "F.Cu") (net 8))
 (segment (start 111.6 115.27) (end 111.6 112.7433) (width 0.3) (layer "F.Cu") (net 8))
 (segment (start 110.5983 111.7416) (end 111.6 112.7433) (width 0.3) (layer "F.Cu") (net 8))
 (segment (start 110.5983 62.9984) (end 110.5983 111.7416) (width 0.3) (layer "F.Cu") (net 8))
 (segment (start 144.62 112.7433) (end 145.6232 111.7401) (width 0.3) (layer "F.Cu") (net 32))
 (segment (start 144.62 115.27) (end 144.62 112.7433) (width 0.3) (layer "F.Cu") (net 32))
 (segment (start 144.62 59.395) (end 144.62 61.9967) (width 0.3) (layer "F.Cu") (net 32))
 (segment (start 145.6232 62.9999) (end 144.62 61.9967) (width 0.3) (layer "F.Cu") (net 32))
 (segment (start 145.6232 111.7401) (end 145.6232 62.9999) (width 0.3) (layer "F.Cu") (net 32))
 (segment (start 147.16 110.9453) (end 147.16 67.245) (width 0.3) (layer "F.Cu") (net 34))
 (segment (start 148.43 120.37) (end 148.43 112.2153) (width 0.3) (layer "F.Cu") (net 34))
 (segment (start 148.43 112.2153) (end 147.16 110.9453) (width 0.3) (layer "F.Cu") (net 34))
 (segment (start 138.27 120.37) (end 138.27 112.9767) (width 0.3) (layer "F.Cu") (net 27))
 (segment (start 137 111.7067) (end 137 67.245) (width 0.3) (layer "F.Cu") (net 27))
 (segment (start 138.27 112.9767) (end 137 111.7067) (width 0.3) (layer "F.Cu") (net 27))
 (segment (start 135.73 120.37) (end 135.73 112.9767) (width 0.3) (layer "F.Cu") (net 25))
 (segment (start 134.46 111.7067) (end 134.46 67.245) (width 0.3) (layer "F.Cu") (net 25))
 (segment (start 135.73 112.9767) (end 134.46 111.7067) (width 0.3) (layer "F.Cu") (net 25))
 (segment (start 107.2 106.06) (end 105.25 108.01) (width 0.3) (layer "F.Cu") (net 3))
 (segment (start 105.25 108.01) (end 105.25 120.37) (width 0.3) (layer "F.Cu") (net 3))
 (segment (start 103.98 67.245) (end 103.98 98.61) (width 0.3) (layer "F.Cu") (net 3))
 (segment (start 107.2 101.83) (end 107.2 106.06) (width 0.3) (layer "F.Cu") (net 3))
 (segment (start 103.98 98.61) (end 107.2 101.83) (width 0.3) (layer "F.Cu") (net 3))
 (segment (start 117.95 71.1167) (end 117.95 120.37) (width 0.3) (layer "F.Cu") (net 13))
 (segment (start 116.68 69.8467) (end 117.95 71.1167) (width 0.3) (layer "F.Cu") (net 13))
 (segment (start 116.68 67.245) (end 116.68 69.8467) (width 0.3) (layer "F.Cu") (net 13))
 (segment (start 139.54 59.395) (end 139.54 61.9967) (width 0.3) (layer "F.Cu") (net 28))
 (segment (start 139.54 115.27) (end 139.54 112.7433) (width 0.3) (layer "F.Cu") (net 28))
 (segment (start 138.5383 62.9984) (end 139.54 61.9967) (width 0.3) (layer "F.Cu") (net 28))
 (segment (start 138.5383 111.7416) (end 138.5383 62.9984) (width 0.3) (layer "F.Cu") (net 28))
 (segment (start 139.54 112.7433) (end 138.5383 111.7416) (width 0.3) (layer "F.Cu") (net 28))
 (segment (start 141.0783 111.7416) (end 141.0783 62.9984) (width 0.3) (layer "F.Cu") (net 30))
 (segment (start 142.08 112.7433) (end 141.0783 111.7416) (width 0.3) (layer "F.Cu") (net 30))
 (segment (start 142.08 59.395) (end 142.08 61.9967) (width 0.3) (layer "F.Cu") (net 30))
 (segment (start 142.08 115.27) (end 142.08 112.7433) (width 0.3) (layer "F.Cu") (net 30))
 (segment (start 141.0783 62.9984) (end 142.08 61.9967) (width 0.3) (layer "F.Cu") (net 30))
 (segment (start 110.0617 111.7416) (end 109.06 112.7433) (width 0.3) (layer "F.Cu") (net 6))
 (segment (start 110.0617 62.9984) (end 110.0617 111.7416) (width 0.3) (layer "F.Cu") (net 6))
 (segment (start 109.06 59.395) (end 109.06 61.9967) (width 0.3) (layer "F.Cu") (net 6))
 (segment (start 109.06 61.9967) (end 110.0617 62.9984) (width 0.3) (layer "F.Cu") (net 6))
 (segment (start 109.06 115.27) (end 109.06 112.7433) (width 0.3) (layer "F.Cu") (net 6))
 (segment (start 129.38 59.395) (end 129.38 61.9967) (width 0.3) (layer "F.Cu") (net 20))
 (segment (start 129.38 115.27) (end 129.38 112.7433) (width 0.3) (layer "F.Cu") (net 20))
 (segment (start 129.38 61.9967) (end 129.38 62.1576) (width 0.3) (layer "F.Cu") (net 20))
 (segment (start 129.38 112.7433) (end 128.172 111.5353) (width 0.3) (layer "F.Cu") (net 20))
 (segment (start 128.172 111.5353) (end 128.172 62.1576) (width 0.3) (layer "F.Cu") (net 20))
 (via (at 128.172 62.1576) (size 0.6) (drill 0.3) (layers "F.Cu" "B.Cu") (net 20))
 (via (at 129.38 62.1576) (size 0.6) (drill 0.3) (layers "F.Cu" "B.Cu") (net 20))
 (segment (start 129.38 62.1576) (end 128.172 62.1576) (width 0.3) (layer "B.Cu") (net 20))
 (segment (start 135.9983 62.9984) (end 137 61.9967) (width 0.3) (layer "F.Cu") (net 26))
 (segment (start 137 115.27) (end 137 112.7433) (width 0.3) (layer "F.Cu") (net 26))
 (segment (start 135.9983 111.7416) (end 135.9983 62.9984) (width 0.3) (layer "F.Cu") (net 26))
 (segment (start 137 112.7433) (end 135.9983 111.7416) (width 0.3) (layer "F.Cu") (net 26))
 (segment (start 137 59.395) (end 137 61.9967) (width 0.3) (layer "F.Cu") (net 26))
 (segment (start 119.22 67.245) (end 119.22 69.8467) (width 0.3) (layer "F.Cu") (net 15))
 (segment (start 120.49 71.1167) (end 119.22 69.8467) (width 0.3) (layer "F.Cu") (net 15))
 (segment (start 120.49 120.37) (end 120.49 71.1167) (width 0.3) (layer "F.Cu") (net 15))
 (segment (start 125.57 120.37) (end 125.57 112.6197) (width 0.3) (layer "F.Cu") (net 17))
 (segment (start 125.57 112.6197) (end 124.3 111.3497) (width 0.3) (layer "F.Cu") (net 17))
 (segment (start 124.3 111.3497) (end 124.3 67.245) (width 0.3) (layer "F.Cu") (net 17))
 (segment (start 115.6783 111.7416) (end 116.68 112.7433) (width 0.3) (layer "F.Cu") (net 12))
 (segment (start 116.68 115.27) (end 116.68 112.7433) (width 0.3) (layer "F.Cu") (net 12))
 (segment (start 116.68 59.395) (end 116.68 61.9967) (width 0.3) (layer "F.Cu") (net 12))
 (segment (start 115.6783 62.9984) (end 115.6783 111.7416) (width 0.3) (layer "F.Cu") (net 12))
 (segment (start 116.68 61.9967) (end 115.6783 62.9984) (width 0.3) (layer "F.Cu") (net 12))
 (segment (start 155.7817 88.6949) (end 153.21 91.2666) (width 0.3) (layer "F.Cu") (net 38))
 (segment (start 154.78 61.9967) (end 155.7817 62.9984) (width 0.3) (layer "F.Cu") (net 38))
 (segment (start 154.78 59.395) (end 154.78 61.9967) (width 0.3) (layer "F.Cu") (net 38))
 (segment (start 153.21 91.2666) (end 153.21 107.0168) (width 0.3) (layer "F.Cu") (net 38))
 (segment (start 154.78 115.27) (end 154.78 112.7433) (width 0.3) (layer "F.Cu") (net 38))
 (segment (start 153.21 107.0168) (end 155.2886 109.0954) (width 0.3) (layer "F.Cu") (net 38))
 (segment (start 153.9325 111.8958) (end 153.9325 110.0042) (width 0.3) (layer "F.Cu") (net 38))
 (segment (start 155.2886 109.0954) (end 155.2886 109.9515) (width 0.3) (layer "F.Cu") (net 38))
 (segment (start 154.78 112.7433) (end 153.9325 111.8958) (width 0.3) (layer "F.Cu") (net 38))
 (segment (start 155.7817 62.9984) (end 155.7817 88.6949) (width 0.3) (layer "F.Cu") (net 38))
 (via (at 155.2886 109.9515) (size 0.6) (drill 0.3) (layers "F.Cu" "B.Cu") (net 38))
 (via (at 153.9325 110.0042) (size 0.6) (drill 0.3) (layers "F.Cu" "B.Cu") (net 38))
 (segment (start 153.9325 110.0042) (end 155.2359 110.0042) (width 0.3) (layer "B.Cu") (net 38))
 (segment (start 155.2359 110.0042) (end 155.2886 109.9515) (width 0.3) (layer "B.Cu") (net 38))
 (segment (start 130.65 120.37) (end 130.65 111.8269) (width 0.3) (layer "F.Cu") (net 21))
 (segment (start 130.65 111.8269) (end 129.38 110.5569) (width 0.3) (layer "F.Cu") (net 21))
 (segment (start 129.38 110.5569) (end 129.38 67.245) (width 0.3) (layer "F.Cu") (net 21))
 (segment (start 130.9183 111.0323) (end 130.9183 62.9984) (width 0.3) (layer "F.Cu") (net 22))
 (segment (start 130.9183 62.9984) (end 131.92 61.9967) (width 0.3) (layer "F.Cu") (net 22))
 (segment (start 131.92 59.395) (end 131.92 61.9967) (width 0.3) (layer "F.Cu") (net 22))
 (segment (start 131.92 115.27) (end 131.92 112.7433) (width 0.3) (layer "F.Cu") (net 22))
 (segment (start 131.92 112.7433) (end 131.92 112.034) (width 0.3) (layer "F.Cu") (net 22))
 (segment (start 131.92 112.034) (end 130.9183 111.0323) (width 0.3) (layer "F.Cu") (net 22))
 (segment (start 115.41 112.5945) (end 114.14 111.3245) (width 0.3) (layer "F.Cu") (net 11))
 (segment (start 114.14 111.3245) (end 114.14 67.245) (width 0.3) (layer "F.Cu") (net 11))
 (segment (start 115.41 120.37) (end 115.41 112.5945) (width 0.3) (layer "F.Cu") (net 11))
 (segment (start 107.9479 112.3321) (end 109.5617 110.7183) (width 0.3) (layer "F.Cu") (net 7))
 (segment (start 109.5617 110.7183) (end 109.5617 70.3484) (width 0.3) (layer "F.Cu") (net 7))
 (segment (start 108.583 117.8433) (end 107.9479 117.2082) (width 0.3) (layer "F.Cu") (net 7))
 (segment (start 109.06 69.8467) (end 109.06 67.245) (width 0.3) (layer "F.Cu") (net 7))
 (segment (start 107.9479 117.2082) (end 107.9479 112.3321) (width 0.3) (layer "F.Cu") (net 7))
 (segment (start 109.5617 70.3484) (end 109.06 69.8467) (width 0.3) (layer "F.Cu") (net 7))
 (segment (start 110.33 117.8433) (end 108.583 117.8433) (width 0.3) (layer "F.Cu") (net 7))
 (segment (start 110.33 120.37) (end 110.33 117.8433) (width 0.3) (layer "F.Cu") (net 7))
 (segment (start 113.1383 111.0323) (end 113.1383 62.9984) (width 0.3) (layer "F.Cu") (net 10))
 (segment (start 114.14 115.27) (end 114.14 112.7433) (width 0.3) (layer "F.Cu") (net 10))
 (segment (start 114.14 59.395) (end 114.14 61.9967) (width 0.3) (layer "F.Cu") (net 10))
 (segment (start 114.14 112.034) (end 113.1383 111.0323) (width 0.3) (layer "F.Cu") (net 10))
 (segment (start 113.1383 62.9984) (end 114.14 61.9967) (width 0.3) (layer "F.Cu") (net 10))
 (segment (start 114.14 112.7433) (end 114.14 112.034) (width 0.3) (layer "F.Cu") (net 10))
 (segment (start 108.05 99.76) (end 108.05 99.85) (width 0.3) (layer "F.Cu") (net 5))
 (segment (start 106.52 98.23) (end 108.05 99.76) (width 0.3) (layer "F.Cu") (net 5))
 (segment (start 107.79 118.05) (end 107.79 120.37) (width 0.3) (layer "F.Cu") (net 5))
 (segment (start 107.45 117.71) (end 107.79 118.05) (width 0.3) (layer "F.Cu") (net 5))
 (segment (start 108.05 99.85) (end 108.05 99.86) (width 0.3) (layer "F.Cu") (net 5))
 (segment (start 106.52 67.245) (end 106.52 98.23) (width 0.3) (layer "F.Cu") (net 5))
 (via (at 108.05 99.85) (size 0.6) (drill 0.3) (layers "F.Cu" "B.Cu") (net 5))
 (via (at 107.45 117.71) (size 0.6) (drill 0.3) (layers "F.Cu" "B.Cu") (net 5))
 (segment (start 107.45 117.71) (end 107.45 117.35) (width 0.3) (layer "B.Cu") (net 5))
 (segment (start 108.74 116.06) (end 108.74 100.54) (width 0.3) (layer "B.Cu") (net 5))
 (segment (start 108.74 100.54) (end 108.05 99.85) (width 0.3) (layer "B.Cu") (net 5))
 (segment (start 107.45 117.35) (end 108.74 116.06) (width 0.3) (layer "B.Cu") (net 5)))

